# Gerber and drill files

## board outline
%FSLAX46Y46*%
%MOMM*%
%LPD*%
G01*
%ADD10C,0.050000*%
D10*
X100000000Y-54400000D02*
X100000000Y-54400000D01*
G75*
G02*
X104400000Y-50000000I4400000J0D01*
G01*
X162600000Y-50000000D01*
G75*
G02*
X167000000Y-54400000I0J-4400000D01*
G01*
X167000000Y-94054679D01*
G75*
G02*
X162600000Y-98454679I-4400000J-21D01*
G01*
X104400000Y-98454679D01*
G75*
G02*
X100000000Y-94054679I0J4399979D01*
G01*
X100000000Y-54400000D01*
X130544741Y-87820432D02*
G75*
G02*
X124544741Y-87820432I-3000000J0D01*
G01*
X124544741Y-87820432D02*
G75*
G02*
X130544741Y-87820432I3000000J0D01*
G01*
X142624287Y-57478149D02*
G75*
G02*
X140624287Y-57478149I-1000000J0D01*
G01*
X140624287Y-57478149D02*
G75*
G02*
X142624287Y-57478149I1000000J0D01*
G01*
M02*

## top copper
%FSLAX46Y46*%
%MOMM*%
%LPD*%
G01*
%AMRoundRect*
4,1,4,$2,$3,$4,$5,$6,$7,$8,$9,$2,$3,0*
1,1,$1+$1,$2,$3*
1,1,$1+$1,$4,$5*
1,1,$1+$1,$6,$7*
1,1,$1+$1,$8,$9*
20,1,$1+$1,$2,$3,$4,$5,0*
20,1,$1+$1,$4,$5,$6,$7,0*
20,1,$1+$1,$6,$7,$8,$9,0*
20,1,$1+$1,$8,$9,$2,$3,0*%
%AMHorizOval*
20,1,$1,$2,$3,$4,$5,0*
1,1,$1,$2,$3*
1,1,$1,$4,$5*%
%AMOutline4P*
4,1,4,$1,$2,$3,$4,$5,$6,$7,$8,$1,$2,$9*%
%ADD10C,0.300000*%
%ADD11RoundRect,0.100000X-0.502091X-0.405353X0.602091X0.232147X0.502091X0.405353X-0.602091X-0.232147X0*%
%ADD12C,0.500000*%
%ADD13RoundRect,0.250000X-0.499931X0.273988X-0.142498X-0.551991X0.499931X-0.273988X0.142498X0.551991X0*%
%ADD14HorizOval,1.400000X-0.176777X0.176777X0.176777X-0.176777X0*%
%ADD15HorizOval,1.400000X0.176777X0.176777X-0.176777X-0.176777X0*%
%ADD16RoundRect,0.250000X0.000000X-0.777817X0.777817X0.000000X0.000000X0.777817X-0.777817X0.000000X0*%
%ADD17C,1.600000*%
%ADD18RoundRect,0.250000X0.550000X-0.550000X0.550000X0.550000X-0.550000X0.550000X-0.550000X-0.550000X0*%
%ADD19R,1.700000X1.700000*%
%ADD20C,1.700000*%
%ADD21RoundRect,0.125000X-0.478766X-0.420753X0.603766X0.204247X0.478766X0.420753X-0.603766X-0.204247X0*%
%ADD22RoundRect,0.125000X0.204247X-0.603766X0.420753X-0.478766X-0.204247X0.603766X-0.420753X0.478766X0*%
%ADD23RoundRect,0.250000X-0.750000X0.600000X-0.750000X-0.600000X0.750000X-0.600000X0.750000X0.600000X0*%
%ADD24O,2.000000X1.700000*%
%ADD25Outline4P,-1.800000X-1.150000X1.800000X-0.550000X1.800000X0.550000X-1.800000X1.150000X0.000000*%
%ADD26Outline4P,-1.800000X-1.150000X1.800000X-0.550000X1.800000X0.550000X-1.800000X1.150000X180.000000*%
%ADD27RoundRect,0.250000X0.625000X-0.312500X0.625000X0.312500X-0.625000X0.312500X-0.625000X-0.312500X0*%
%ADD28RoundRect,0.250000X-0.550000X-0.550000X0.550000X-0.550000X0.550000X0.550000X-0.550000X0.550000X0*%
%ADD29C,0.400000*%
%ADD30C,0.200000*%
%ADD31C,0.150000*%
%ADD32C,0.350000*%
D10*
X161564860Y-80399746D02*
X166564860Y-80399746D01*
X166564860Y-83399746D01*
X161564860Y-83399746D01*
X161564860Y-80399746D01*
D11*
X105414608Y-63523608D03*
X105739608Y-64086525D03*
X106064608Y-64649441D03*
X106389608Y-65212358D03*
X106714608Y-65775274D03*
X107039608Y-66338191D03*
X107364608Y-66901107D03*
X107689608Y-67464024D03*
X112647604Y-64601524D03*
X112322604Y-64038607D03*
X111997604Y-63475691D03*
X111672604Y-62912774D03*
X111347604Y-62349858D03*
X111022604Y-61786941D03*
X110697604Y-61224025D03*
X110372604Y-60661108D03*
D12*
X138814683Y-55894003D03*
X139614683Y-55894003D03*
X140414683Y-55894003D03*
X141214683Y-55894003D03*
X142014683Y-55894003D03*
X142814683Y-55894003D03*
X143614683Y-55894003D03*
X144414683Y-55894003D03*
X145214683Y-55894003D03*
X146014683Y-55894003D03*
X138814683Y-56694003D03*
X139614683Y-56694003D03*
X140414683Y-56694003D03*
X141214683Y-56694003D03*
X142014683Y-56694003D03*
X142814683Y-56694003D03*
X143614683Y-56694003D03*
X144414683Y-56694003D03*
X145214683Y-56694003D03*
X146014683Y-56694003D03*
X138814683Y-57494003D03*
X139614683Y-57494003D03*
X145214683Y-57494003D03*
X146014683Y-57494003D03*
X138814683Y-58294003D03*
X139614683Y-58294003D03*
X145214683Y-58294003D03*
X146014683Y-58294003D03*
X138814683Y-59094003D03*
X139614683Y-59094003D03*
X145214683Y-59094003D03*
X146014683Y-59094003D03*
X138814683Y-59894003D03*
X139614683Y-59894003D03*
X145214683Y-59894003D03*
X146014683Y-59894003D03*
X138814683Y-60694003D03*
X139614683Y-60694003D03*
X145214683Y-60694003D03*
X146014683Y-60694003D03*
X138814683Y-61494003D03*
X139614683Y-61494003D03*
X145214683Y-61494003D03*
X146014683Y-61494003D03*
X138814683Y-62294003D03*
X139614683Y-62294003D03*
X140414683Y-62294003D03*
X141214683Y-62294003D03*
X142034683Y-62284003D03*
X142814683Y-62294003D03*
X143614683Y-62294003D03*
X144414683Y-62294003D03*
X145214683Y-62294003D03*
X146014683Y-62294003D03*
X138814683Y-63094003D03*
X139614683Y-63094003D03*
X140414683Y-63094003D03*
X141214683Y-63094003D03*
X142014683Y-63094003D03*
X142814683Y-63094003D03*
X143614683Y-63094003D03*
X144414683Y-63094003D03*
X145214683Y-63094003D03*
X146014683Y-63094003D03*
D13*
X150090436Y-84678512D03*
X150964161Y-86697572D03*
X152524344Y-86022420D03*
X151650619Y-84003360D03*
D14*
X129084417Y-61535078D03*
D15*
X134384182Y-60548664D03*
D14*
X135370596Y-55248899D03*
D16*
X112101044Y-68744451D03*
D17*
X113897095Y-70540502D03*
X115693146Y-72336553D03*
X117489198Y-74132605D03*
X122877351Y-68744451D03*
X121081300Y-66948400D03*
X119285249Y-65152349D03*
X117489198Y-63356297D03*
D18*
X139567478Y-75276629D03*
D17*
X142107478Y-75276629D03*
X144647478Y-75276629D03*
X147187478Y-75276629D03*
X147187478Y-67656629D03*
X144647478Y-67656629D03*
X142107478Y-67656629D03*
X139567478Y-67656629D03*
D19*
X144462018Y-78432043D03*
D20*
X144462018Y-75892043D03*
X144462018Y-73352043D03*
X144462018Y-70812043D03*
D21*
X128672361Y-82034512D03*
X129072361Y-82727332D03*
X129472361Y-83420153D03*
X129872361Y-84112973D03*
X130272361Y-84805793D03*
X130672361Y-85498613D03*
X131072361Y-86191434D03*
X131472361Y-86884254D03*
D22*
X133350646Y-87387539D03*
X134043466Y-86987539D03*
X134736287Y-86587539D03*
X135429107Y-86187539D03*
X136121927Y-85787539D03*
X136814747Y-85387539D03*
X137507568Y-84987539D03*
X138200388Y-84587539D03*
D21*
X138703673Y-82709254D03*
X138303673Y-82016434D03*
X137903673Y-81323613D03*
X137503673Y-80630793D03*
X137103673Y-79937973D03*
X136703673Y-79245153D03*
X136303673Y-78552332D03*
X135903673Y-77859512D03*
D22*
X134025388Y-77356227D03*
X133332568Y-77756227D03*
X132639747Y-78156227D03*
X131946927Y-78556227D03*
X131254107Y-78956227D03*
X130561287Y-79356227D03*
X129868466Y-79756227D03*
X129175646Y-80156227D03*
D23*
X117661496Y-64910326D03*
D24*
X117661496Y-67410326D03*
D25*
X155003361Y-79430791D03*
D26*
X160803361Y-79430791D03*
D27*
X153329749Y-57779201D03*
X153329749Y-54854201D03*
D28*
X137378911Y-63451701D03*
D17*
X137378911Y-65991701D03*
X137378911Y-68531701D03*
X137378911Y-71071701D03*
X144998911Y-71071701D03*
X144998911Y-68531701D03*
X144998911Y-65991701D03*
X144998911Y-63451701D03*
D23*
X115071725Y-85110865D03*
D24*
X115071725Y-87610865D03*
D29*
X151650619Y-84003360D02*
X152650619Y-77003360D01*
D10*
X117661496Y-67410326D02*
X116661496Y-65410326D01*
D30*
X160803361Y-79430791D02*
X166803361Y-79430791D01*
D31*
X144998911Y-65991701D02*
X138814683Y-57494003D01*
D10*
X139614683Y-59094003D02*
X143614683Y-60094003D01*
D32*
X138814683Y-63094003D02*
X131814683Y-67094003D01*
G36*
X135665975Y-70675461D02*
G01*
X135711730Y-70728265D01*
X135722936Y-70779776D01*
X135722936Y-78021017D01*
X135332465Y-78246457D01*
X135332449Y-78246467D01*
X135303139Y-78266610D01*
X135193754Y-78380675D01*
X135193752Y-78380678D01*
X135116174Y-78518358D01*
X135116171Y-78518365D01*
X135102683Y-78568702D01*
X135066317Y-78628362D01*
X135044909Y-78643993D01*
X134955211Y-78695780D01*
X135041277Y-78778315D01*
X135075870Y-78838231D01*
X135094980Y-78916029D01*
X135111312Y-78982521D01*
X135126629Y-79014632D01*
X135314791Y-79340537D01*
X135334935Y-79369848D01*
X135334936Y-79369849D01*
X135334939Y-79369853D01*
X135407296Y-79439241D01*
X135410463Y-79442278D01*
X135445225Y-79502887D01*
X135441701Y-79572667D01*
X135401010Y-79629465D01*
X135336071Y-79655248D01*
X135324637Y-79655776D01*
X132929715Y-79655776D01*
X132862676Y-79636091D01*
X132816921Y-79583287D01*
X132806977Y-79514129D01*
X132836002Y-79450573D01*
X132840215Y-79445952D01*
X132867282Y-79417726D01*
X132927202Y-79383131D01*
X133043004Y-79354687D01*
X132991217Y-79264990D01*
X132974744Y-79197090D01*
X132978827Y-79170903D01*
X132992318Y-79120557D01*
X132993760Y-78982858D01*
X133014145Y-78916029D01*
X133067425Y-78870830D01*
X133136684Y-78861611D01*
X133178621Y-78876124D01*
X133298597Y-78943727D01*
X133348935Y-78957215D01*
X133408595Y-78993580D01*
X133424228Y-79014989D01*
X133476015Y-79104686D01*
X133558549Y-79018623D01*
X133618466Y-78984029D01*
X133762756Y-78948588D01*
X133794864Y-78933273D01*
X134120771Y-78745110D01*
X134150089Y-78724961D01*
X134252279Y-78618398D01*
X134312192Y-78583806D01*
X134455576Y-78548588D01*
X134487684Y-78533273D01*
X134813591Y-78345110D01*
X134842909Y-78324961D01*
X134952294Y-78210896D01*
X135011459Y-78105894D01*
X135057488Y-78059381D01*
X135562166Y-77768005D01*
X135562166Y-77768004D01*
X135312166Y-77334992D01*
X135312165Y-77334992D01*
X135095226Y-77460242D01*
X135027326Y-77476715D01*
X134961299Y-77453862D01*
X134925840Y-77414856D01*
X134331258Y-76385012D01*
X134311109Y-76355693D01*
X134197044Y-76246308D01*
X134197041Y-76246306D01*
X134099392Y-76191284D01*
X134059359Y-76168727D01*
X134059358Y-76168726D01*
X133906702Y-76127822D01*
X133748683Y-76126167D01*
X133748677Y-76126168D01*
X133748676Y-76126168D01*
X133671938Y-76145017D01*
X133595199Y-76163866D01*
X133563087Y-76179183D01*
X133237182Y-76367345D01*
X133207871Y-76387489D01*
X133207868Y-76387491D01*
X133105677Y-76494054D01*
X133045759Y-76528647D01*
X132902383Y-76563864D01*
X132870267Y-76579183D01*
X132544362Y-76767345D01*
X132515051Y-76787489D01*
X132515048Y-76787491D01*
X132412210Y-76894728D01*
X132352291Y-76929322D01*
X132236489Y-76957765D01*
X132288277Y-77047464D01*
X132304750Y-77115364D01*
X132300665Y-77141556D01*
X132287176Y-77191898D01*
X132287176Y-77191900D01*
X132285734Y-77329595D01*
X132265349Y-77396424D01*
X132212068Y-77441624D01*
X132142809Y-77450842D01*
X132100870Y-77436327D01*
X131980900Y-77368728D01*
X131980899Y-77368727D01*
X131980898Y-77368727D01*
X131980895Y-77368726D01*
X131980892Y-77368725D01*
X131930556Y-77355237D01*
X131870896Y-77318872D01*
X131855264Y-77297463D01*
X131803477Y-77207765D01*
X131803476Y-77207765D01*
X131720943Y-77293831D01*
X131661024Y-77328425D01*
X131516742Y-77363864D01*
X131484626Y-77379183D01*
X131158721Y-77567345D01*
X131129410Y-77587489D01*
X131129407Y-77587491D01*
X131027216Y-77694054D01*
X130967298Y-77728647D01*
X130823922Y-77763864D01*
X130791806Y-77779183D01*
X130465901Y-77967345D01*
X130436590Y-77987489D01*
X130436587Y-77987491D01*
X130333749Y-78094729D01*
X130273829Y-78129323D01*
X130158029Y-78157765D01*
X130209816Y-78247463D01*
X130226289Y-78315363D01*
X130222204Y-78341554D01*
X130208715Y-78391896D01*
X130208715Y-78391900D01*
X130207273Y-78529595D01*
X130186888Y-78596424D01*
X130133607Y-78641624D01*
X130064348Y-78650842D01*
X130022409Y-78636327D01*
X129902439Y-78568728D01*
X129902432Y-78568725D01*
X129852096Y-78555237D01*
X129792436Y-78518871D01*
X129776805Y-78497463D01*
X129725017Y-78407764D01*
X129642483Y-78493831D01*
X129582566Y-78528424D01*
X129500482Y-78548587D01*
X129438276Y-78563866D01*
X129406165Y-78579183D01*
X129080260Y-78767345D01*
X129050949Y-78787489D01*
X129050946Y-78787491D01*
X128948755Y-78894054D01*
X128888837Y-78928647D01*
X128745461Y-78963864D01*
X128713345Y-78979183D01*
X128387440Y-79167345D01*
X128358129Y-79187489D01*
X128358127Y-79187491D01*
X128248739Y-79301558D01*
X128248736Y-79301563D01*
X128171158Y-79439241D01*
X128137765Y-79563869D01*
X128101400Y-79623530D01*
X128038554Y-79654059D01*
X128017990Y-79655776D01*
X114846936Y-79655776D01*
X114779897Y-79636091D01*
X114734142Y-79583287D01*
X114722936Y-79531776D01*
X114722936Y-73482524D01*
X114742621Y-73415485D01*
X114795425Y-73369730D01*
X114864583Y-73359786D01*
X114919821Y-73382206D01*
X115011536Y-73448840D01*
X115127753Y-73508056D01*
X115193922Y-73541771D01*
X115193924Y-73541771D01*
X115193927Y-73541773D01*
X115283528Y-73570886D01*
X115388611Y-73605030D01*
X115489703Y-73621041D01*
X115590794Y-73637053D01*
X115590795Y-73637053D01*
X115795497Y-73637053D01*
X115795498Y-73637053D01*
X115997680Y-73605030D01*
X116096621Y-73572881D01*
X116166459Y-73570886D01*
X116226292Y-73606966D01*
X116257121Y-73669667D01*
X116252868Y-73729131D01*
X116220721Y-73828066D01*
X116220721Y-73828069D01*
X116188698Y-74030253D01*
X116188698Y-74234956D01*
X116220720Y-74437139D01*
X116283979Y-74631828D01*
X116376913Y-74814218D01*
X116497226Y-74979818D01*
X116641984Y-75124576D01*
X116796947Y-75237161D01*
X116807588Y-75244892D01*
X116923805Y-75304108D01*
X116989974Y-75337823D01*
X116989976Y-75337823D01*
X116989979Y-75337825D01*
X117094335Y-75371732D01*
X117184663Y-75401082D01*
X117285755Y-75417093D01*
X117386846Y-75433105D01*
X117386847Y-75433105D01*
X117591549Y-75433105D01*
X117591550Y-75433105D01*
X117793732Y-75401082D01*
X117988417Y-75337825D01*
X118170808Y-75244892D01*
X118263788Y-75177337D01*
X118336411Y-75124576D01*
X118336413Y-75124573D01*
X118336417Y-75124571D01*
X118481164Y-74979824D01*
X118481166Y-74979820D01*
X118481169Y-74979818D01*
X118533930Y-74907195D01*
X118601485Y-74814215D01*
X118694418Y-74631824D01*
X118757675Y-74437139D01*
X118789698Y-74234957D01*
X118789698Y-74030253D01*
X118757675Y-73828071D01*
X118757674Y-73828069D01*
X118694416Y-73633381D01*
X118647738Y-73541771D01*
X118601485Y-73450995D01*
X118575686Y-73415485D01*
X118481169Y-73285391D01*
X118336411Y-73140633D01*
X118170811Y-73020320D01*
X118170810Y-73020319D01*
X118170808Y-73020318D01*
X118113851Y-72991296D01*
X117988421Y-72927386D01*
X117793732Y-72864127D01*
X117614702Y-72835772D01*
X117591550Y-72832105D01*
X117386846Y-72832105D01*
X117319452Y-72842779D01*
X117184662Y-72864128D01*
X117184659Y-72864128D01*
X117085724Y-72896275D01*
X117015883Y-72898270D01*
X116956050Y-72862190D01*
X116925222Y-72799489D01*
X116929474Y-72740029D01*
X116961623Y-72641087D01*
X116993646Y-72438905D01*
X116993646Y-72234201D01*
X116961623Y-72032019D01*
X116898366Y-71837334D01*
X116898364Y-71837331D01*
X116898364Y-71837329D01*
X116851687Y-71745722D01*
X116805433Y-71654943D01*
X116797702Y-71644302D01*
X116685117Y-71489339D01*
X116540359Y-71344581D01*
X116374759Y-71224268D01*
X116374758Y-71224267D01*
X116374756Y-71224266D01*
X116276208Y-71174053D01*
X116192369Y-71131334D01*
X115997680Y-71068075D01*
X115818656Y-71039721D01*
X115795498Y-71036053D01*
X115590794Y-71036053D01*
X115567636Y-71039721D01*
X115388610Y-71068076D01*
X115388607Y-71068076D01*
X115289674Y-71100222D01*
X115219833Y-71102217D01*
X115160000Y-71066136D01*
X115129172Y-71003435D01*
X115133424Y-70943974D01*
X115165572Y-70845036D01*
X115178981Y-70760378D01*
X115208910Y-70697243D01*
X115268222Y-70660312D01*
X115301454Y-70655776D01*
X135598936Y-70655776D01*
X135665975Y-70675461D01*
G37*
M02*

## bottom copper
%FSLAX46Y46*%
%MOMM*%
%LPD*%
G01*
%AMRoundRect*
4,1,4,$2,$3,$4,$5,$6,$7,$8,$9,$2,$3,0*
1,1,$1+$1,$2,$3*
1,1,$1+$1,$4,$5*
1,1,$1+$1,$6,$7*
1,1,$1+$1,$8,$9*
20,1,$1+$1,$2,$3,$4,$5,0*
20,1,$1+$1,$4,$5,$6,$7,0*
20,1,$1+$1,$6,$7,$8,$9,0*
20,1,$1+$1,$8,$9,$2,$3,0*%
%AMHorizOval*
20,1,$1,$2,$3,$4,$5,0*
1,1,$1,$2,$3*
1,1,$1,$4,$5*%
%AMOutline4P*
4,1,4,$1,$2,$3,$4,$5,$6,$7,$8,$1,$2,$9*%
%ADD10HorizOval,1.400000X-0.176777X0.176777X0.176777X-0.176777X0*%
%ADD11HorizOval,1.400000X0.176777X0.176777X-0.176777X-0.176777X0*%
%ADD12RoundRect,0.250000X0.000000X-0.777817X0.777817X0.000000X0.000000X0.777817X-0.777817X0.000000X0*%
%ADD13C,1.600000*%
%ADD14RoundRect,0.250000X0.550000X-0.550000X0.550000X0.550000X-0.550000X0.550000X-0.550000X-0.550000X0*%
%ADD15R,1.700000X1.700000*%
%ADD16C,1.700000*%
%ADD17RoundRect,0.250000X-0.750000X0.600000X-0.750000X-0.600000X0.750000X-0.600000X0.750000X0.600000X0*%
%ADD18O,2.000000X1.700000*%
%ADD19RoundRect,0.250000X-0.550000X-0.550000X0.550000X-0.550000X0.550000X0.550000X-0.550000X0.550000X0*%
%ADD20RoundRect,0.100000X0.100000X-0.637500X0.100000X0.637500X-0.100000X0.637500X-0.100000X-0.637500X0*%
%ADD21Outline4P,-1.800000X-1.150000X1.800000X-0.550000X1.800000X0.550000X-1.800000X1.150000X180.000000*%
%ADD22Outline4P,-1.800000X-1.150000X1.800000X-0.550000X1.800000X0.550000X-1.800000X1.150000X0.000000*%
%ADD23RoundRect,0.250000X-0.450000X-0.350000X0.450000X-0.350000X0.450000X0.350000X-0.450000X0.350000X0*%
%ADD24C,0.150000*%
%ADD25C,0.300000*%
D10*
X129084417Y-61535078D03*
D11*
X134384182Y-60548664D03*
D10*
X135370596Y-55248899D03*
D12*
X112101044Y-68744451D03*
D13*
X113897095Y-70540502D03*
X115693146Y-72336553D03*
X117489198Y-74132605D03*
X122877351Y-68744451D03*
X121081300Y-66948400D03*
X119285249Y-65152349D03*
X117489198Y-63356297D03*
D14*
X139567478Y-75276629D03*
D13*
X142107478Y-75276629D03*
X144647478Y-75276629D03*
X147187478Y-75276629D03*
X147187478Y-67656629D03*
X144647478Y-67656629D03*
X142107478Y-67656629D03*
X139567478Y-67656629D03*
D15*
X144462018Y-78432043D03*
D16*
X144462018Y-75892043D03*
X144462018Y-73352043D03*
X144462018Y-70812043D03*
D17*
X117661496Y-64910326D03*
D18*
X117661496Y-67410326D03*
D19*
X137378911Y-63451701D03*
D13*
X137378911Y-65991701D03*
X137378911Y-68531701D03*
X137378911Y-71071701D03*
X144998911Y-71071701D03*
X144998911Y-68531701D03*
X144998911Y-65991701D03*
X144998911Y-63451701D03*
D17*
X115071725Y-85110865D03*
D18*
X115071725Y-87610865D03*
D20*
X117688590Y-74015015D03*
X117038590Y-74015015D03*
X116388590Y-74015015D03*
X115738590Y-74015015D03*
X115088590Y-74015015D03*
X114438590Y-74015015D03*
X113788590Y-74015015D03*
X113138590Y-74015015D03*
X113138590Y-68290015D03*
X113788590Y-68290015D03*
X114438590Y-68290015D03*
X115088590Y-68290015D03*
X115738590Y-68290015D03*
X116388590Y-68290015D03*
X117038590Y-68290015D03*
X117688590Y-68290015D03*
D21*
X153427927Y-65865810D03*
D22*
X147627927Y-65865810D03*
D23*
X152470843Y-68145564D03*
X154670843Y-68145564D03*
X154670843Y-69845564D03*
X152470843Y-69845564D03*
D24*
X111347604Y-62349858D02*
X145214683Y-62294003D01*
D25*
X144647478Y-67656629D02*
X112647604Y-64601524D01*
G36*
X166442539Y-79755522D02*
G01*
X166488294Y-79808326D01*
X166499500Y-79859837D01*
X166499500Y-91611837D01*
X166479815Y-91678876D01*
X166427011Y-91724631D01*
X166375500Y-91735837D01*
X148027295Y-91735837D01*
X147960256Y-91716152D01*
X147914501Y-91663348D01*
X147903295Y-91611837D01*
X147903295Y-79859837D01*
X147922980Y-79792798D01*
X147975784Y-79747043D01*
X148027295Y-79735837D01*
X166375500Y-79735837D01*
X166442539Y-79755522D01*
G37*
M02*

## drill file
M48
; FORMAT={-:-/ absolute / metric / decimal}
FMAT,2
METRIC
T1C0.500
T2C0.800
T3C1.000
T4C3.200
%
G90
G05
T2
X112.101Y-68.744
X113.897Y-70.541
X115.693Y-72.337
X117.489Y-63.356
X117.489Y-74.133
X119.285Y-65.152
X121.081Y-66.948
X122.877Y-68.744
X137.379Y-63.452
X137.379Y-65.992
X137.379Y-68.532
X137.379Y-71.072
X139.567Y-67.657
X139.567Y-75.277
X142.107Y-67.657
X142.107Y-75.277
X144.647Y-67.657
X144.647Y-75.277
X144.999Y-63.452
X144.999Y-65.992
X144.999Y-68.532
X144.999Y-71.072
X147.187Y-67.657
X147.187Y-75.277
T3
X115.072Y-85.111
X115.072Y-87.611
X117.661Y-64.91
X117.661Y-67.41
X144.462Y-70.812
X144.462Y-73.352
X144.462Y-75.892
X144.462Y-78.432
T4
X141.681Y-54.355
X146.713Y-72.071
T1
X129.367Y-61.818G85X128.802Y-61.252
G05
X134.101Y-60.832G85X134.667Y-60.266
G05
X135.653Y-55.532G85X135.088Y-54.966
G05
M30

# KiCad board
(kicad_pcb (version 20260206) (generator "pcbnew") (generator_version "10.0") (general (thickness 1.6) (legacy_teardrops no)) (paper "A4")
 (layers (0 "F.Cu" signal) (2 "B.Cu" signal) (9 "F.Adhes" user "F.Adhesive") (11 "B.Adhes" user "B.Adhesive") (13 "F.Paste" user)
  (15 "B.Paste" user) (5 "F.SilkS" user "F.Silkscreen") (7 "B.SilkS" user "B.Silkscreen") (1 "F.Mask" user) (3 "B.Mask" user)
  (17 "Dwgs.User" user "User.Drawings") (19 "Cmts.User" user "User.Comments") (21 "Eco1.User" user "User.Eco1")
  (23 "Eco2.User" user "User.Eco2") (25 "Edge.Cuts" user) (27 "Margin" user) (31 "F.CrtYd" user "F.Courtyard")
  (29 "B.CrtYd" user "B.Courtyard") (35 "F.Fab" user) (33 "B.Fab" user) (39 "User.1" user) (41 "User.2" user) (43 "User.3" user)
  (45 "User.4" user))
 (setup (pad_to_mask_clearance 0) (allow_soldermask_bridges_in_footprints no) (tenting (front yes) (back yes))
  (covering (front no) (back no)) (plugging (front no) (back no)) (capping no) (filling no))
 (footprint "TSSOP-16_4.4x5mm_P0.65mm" (layer "F.Cu") (at 109.031106 64.062566 30)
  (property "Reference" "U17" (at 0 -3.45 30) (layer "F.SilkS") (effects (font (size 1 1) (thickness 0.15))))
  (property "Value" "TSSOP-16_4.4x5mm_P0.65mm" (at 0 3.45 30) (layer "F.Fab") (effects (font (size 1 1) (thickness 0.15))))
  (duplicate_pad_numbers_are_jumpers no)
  (pad "1" smd roundrect (at -2.8625 -2.275 30) (size 1.475 0.4) (layers "F.Cu" "F.Mask" "F.Paste") (roundrect_rratio 0.25))
  (pad "2" smd roundrect (at -2.8625 -1.625 30) (size 1.475 0.4) (layers "F.Cu" "F.Mask" "F.Paste") (roundrect_rratio 0.25) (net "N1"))
  (pad "3" smd roundrect (at -2.8625 -0.975 30) (size 1.475 0.4) (layers "F.Cu" "F.Mask" "F.Paste") (roundrect_rratio 0.25) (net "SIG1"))
  (pad "4" smd roundrect (at -2.8625 -0.325 30) (size 1.475 0.4) (layers "F.Cu" "F.Mask" "F.Paste") (roundrect_rratio 0.25) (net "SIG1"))
  (pad "5" smd roundrect (at -2.8625 0.325 30) (size 1.475 0.4) (layers "F.Cu" "F.Mask" "F.Paste") (roundrect_rratio 0.25) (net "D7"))
  (pad "6" smd roundrect (at -2.8625 0.975 30) (size 1.475 0.4) (layers "F.Cu" "F.Mask" "F.Paste") (roundrect_rratio 0.25) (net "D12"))
  (pad "7" smd roundrect (at -2.8625 1.625 30) (size 1.475 0.4) (layers "F.Cu" "F.Mask" "F.Paste") (roundrect_rratio 0.25))
  (pad "8" smd roundrect (at -2.8625 2.275 30) (size 1.475 0.4) (layers "F.Cu" "F.Mask" "F.Paste") (roundrect_rratio 0.25) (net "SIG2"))
  (pad "9" smd roundrect (at 2.8625 2.275 30) (size 1.475 0.4) (layers "F.Cu" "F.Mask" "F.Paste") (roundrect_rratio 0.25) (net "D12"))
  (pad "10" smd roundrect (at 2.8625 1.625 30) (size 1.475 0.4) (layers "F.Cu" "F.Mask" "F.Paste") (roundrect_rratio 0.25) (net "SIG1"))
  (pad "11" smd roundrect (at 2.8625 0.975 30) (size 1.475 0.4) (layers "F.Cu" "F.Mask" "F.Paste") (roundrect_rratio 0.25) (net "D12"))
  (pad "12" smd roundrect (at 2.8625 0.325 30) (size 1.475 0.4) (layers "F.Cu" "F.Mask" "F.Paste") (roundrect_rratio 0.25))
  (pad "13" smd roundrect (at 2.8625 -0.325 30) (size 1.475 0.4) (layers "F.Cu" "F.Mask" "F.Paste") (roundrect_rratio 0.25))
  (pad "14" smd roundrect (at 2.8625 -0.975 30) (size 1.475 0.4) (layers "F.Cu" "F.Mask" "F.Paste") (roundrect_rratio 0.25) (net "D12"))
  (pad "15" smd roundrect (at 2.8625 -1.625 30) (size 1.475 0.4) (layers "F.Cu" "F.Mask" "F.Paste") (roundrect_rratio 0.25) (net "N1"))
  (pad "16" smd roundrect (at 2.8625 -2.275 30) (size 1.475 0.4) (layers "F.Cu" "F.Mask" "F.Paste") (roundrect_rratio 0.25) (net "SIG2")))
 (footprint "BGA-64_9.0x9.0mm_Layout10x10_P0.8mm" (layer "F.Cu") (at 142.414683 59.494003)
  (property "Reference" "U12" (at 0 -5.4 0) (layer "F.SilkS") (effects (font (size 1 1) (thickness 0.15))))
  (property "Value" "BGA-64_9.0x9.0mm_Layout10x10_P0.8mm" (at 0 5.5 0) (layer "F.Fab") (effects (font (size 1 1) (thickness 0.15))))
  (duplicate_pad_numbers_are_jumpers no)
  (pad "A1" smd circle (at -3.6 -3.6) (size 0.5 0.5) (layers "F.Cu" "F.Mask" "F.Paste") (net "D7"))
  (pad "A2" smd circle (at -2.8 -3.6) (size 0.5 0.5) (layers "F.Cu" "F.Mask" "F.Paste") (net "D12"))
  (pad "A3" smd circle (at -2 -3.6) (size 0.5 0.5) (layers "F.Cu" "F.Mask" "F.Paste"))
  (pad "A4" smd circle (at -1.2 -3.6) (size 0.5 0.5) (layers "F.Cu" "F.Mask" "F.Paste") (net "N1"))
  (pad "A5" smd circle (at -0.4 -3.6) (size 0.5 0.5) (layers "F.Cu" "F.Mask" "F.Paste") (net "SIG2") (clearance 0.35))
  (pad "A6" smd circle (at 0.4 -3.6) (size 0.5 0.5) (layers "F.Cu" "F.Mask" "F.Paste"))
  (pad "A7" smd circle (at 1.2 -3.6) (size 0.5 0.5) (layers "F.Cu" "F.Mask" "F.Paste") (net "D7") (clearance 0.1))
  (pad "A8" smd circle (at 2 -3.6) (size 0.5 0.5) (layers "F.Cu" "F.Mask" "F.Paste") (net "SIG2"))
  (pad "A9" smd circle (at 2.8 -3.6) (size 0.5 0.5) (layers "F.Cu" "F.Mask" "F.Paste") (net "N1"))
  (pad "A10" smd circle (at 3.6 -3.6) (size 0.5 0.5) (layers "F.Cu" "F.Mask" "F.Paste"))
  (pad "B1" smd circle (at -3.6 -2.8) (size 0.5 0.5) (layers "F.Cu" "F.Mask" "F.Paste") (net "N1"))
  (pad "B2" smd circle (at -2.8 -2.8) (size 0.5 0.5) (layers "F.Cu" "F.Mask" "F.Paste") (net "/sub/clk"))
  (pad "B3" smd circle (at -2 -2.8) (size 0.5 0.5) (layers "F.Cu" "F.Mask" "F.Paste") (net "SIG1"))
  (pad "B4" smd circle (at -1.2 -2.8) (size 0.5 0.5) (layers "F.Cu" "F.Mask" "F.Paste"))
  (pad "B5" smd circle (at -0.4 -2.8) (size 0.5 0.5) (layers "F.Cu" "F.Mask" "F.Paste"))
  (pad "B6" smd circle (at 0.4 -2.8) (size 0.5 0.5) (layers "F.Cu" "F.Mask" "F.Paste") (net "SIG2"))
  (pad "B7" smd circle (at 1.2 -2.8) (size 0.5 0.5) (layers "F.Cu" "F.Mask" "F.Paste"))
  (pad "B8" smd circle (at 2 -2.8) (size 0.5 0.5) (layers "F.Cu" "F.Mask" "F.Paste"))
  (pad "B9" smd circle (at 2.8 -2.8) (size 0.5 0.5) (layers "F.Cu" "F.Mask" "F.Paste"))
  (pad "B10" smd circle (at 3.6 -2.8) (size 0.5 0.5) (layers "F.Cu" "F.Mask" "F.Paste") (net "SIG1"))
  (pad "C1" smd circle (at -3.6 -2) (size 0.5 0.5) (layers "F.Cu" "F.Mask" "F.Paste") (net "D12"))
  (pad "C2" smd circle (at -2.8 -2) (size 0.5 0.5) (layers "F.Cu" "F.Mask" "F.Paste") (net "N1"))
  (pad "C9" smd circle (at 2.8 -2) (size 0.5 0.5) (layers "F.Cu" "F.Mask" "F.Paste"))
  (pad "C10" smd circle (at 3.6 -2) (size 0.5 0.5) (layers "F.Cu" "F.Mask" "F.Paste") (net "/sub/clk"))
  (pad "D1" smd circle (at -3.6 -1.2) (size 0.5 0.5) (layers "F.Cu" "F.Mask" "F.Paste") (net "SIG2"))
  (pad "D2" smd circle (at -2.8 -1.2) (size 0.5 0.5) (layers "F.Cu" "F.Mask" "F.Paste"))
  (pad "D9" smd circle (at 2.8 -1.2) (size 0.5 0.5) (layers "F.Cu" "F.Mask" "F.Paste") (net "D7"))
  (pad "D10" smd circle (at 3.6 -1.2) (size 0.5 0.5) (layers "F.Cu" "F.Mask" "F.Paste") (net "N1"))
  (pad "E1" smd circle (at -3.6 -0.4) (size 0.5 0.5) (layers "F.Cu" "F.Mask" "F.Paste") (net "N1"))
  (pad "E2" smd circle (at -2.8 -0.4) (size 0.5 0.5) (layers "F.Cu" "F.Mask" "F.Paste") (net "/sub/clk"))
  (pad "E9" smd circle (at 2.8 -0.4) (size 0.5 0.5) (layers "F.Cu" "F.Mask" "F.Paste") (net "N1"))
  (pad "E10" smd circle (at 3.6 -0.4) (size 0.5 0.5) (layers "F.Cu" "F.Mask" "F.Paste"))
  (pad "F1" smd circle (at -3.6 0.4) (size 0.5 0.5) (layers "F.Cu" "F.Mask" "F.Paste") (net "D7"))
  (pad "F2" smd circle (at -2.8 0.4) (size 0.5 0.5) (layers "F.Cu" "F.Mask" "F.Paste") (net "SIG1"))
  (pad "F9" smd circle (at 2.8 0.4) (size 0.5 0.5) (layers "F.Cu" "F.Mask" "F.Paste"))
  (pad "F10" smd circle (at 3.6 0.4) (size 0.5 0.5) (layers "F.Cu" "F.Mask" "F.Paste") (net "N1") (clearance 0.1))
  (pad "G1" smd circle (at -3.6 1.2) (size 0.5 0.5) (layers "F.Cu" "F.Mask" "F.Paste") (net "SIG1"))
  (pad "G2" smd circle (at -2.8 1.2) (size 0.5 0.5) (layers "F.Cu" "F.Mask" "F.Paste"))
  (pad "G9" smd circle (at 2.8 1.2) (size 0.5 0.5) (layers "F.Cu" "F.Mask" "F.Paste"))
  (pad "G10" smd circle (at 3.6 1.2) (size 0.5 0.5) (layers "F.Cu" "F.Mask" "F.Paste"))
  (pad "H1" smd circle (at -3.6 2) (size 0.5 0.5) (layers "F.Cu" "F.Mask" "F.Paste") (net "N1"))
  (pad "H2" smd circle (at -2.8 2) (size 0.5 0.5) (layers "F.Cu" "F.Mask" "F.Paste"))
  (pad "H9" smd circle (at 2.8 2) (size 0.5 0.5) (layers "F.Cu" "F.Mask" "F.Paste") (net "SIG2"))
  (pad "H10" smd circle (at 3.6 2) (size 0.5 0.5) (layers "F.Cu" "F.Mask" "F.Paste") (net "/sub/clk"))
  (pad "J1" smd circle (at -3.6 2.8) (size 0.5 0.5) (layers "F.Cu" "F.Mask" "F.Paste") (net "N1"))
  (pad "J2" smd circle (at -2.8 2.8) (size 0.5 0.5) (layers "F.Cu" "F.Mask" "F.Paste") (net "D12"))
  (pad "J3" smd circle (at -2 2.8) (size 0.5 0.5) (layers "F.Cu" "F.Mask" "F.Paste") (clearance 0.35))
  (pad "J4" smd circle (at -1.2 2.8) (size 0.5 0.5) (layers "F.Cu" "F.Mask" "F.Paste") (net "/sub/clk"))
  (pad "J5" smd circle (at -0.38 2.79) (size 0.5 0.5) (layers "F.Cu" "F.Mask" "F.Paste") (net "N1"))
  (pad "J6" smd circle (at 0.4 2.8) (size 0.5 0.5) (layers "F.Cu" "F.Mask" "F.Paste") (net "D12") (clearance 0.35))
  (pad "J7" smd circle (at 1.2 2.8) (size 0.5 0.5) (layers "F.Cu" "F.Mask" "F.Paste"))
  (pad "J8" smd circle (at 2 2.8) (size 0.5 0.5) (layers "F.Cu" "F.Mask" "F.Paste") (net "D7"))
  (pad "J9" smd circle (at 2.8 2.8) (size 0.5 0.5) (layers "F.Cu" "F.Mask" "F.Paste") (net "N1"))
  (pad "J10" smd circle (at 3.6 2.8) (size 0.5 0.5) (layers "F.Cu" "F.Mask" "F.Paste") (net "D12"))
  (pad "K1" smd circle (at -3.6 3.6) (size 0.5 0.5) (layers "F.Cu" "F.Mask" "F.Paste") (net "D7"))
  (pad "K2" smd circle (at -2.8 3.6) (size 0.5 0.5) (layers "F.Cu" "F.Mask" "F.Paste"))
  (pad "K3" smd circle (at -2 3.6) (size 0.5 0.5) (layers "F.Cu" "F.Mask" "F.Paste") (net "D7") (clearance 0.35))
  (pad "K4" smd circle (at -1.2 3.6) (size 0.5 0.5) (layers "F.Cu" "F.Mask" "F.Paste") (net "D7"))
  (pad "K5" smd circle (at -0.4 3.6) (size 0.5 0.5) (layers "F.Cu" "F.Mask" "F.Paste") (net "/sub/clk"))
  (pad "K6" smd circle (at 0.4 3.6) (size 0.5 0.5) (layers "F.Cu" "F.Mask" "F.Paste") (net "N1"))
  (pad "K7" smd circle (at 1.2 3.6) (size 0.5 0.5) (layers "F.Cu" "F.Mask" "F.Paste"))
  (pad "K8" smd circle (at 2 3.6) (size 0.5 0.5) (layers "F.Cu" "F.Mask" "F.Paste") (clearance 0.1))
  (pad "K9" smd circle (at 2.8 3.6) (size 0.5 0.5) (layers "F.Cu" "F.Mask" "F.Paste") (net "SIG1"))
  (pad "K10" smd circle (at 3.6 3.6) (size 0.5 0.5) (layers "F.Cu" "F.Mask" "F.Paste") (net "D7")))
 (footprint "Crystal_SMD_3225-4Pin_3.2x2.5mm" (layer "F.Cu") (at 151.30739 85.350466 -66.6)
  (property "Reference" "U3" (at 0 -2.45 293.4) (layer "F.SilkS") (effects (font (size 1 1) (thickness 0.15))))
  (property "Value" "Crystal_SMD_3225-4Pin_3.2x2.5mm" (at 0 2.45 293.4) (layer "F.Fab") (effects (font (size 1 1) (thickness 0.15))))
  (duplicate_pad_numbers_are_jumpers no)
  (pad "1" smd roundrect (at -1.1 0.85 293.4) (size 1.4 1.2) (layers "F.Cu" "F.Mask" "F.Paste") (roundrect_rratio 0.208333) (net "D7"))
  (pad "2" smd roundrect (at 1.1 0.85 293.4) (size 1.4 1.2) (layers "F.Cu" "F.Mask" "F.Paste") (roundrect_rratio 0.208333))
  (pad "3" smd roundrect (at 1.1 -0.85 293.4) (size 1.4 1.2) (layers "F.Cu" "F.Mask" "F.Paste") (roundrect_rratio 0.208333) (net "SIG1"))
  (pad "4" smd roundrect (at -1.1 -0.85 293.4) (size 1.4 1.2) (layers "F.Cu" "F.Mask" "F.Paste") (roundrect_rratio 0.208333)))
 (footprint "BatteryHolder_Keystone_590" (layer "F.Cu") (at 134.384182 60.548664 45)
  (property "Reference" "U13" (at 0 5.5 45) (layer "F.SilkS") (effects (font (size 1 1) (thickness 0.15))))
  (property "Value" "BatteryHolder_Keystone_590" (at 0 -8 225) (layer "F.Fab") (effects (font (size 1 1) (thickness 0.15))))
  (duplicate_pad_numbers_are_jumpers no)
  (pad "1" thru_hole oval (at -4.445 -3.05 135) (size 1.9 1.4) (drill oval 1.3 0.5) (layers "*.Cu" "*.Mask") (remove_unused_layers no)
   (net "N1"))
  (pad "1" thru_hole oval (at 0 0 45) (size 1.9 1.4) (drill oval 1.3 0.5) (layers "*.Cu" "*.Mask") (remove_unused_layers no) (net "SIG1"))
  (pad "1" thru_hole oval (at 4.445 -3.05 135) (size 1.9 1.4) (drill oval 1.3 0.5) (layers "*.Cu" "*.Mask") (remove_unused_layers no)
   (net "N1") (clearance 0.35)))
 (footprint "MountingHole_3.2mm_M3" (layer "F.Cu") (at 146.713095 72.070667 45)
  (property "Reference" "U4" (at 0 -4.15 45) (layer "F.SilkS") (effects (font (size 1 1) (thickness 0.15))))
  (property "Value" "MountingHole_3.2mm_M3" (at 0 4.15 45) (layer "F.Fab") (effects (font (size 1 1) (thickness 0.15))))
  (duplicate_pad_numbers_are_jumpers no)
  (pad "" np_thru_hole circle (at 0 0 45) (size 3.2 3.2) (drill 3.2) (layers "*.Cu" "*.Mask")))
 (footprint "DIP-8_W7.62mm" (layer "F.Cu") (at 112.101044 68.744451 45)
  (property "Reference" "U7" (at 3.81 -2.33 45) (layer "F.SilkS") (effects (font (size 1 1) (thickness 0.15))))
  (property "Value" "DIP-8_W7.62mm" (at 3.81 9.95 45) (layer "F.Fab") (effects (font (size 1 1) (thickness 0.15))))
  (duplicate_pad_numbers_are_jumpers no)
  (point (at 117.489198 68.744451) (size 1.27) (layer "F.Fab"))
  (pad "1" thru_hole roundrect (at 0 0 45) (size 1.6 1.6) (drill 0.8) (layers "*.Cu" "*.Mask") (remove_unused_layers no)
   (roundrect_rratio 0.15625) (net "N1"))
  (pad "2" thru_hole circle (at 0 2.54 45) (size 1.6 1.6) (drill 0.8) (layers "*.Cu" "*.Mask") (remove_unused_layers no))
  (pad "3" thru_hole circle (at 0 5.079999 45) (size 1.6 1.6) (drill 0.8) (layers "*.Cu" "*.Mask") (remove_unused_layers no) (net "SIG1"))
  (pad "4" thru_hole circle (at 0 7.62 45) (size 1.6 1.6) (drill 0.8) (layers "*.Cu" "*.Mask") (remove_unused_layers no) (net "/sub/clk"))
  (pad "5" thru_hole circle (at 7.62 7.62 45) (size 1.6 1.6) (drill 0.8) (layers "*.Cu" "*.Mask") (remove_unused_layers no) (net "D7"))
  (pad "6" thru_hole circle (at 7.62 5.08 45) (size 1.6 1.6) (drill 0.8) (layers "*.Cu" "*.Mask") (remove_unused_layers no))
  (pad "7" thru_hole circle (at 7.62 2.54 45) (size 1.6 1.6) (drill 0.8) (layers "*.Cu" "*.Mask") (remove_unused_layers no) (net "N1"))
  (pad "8" thru_hole circle (at 7.62 0 45) (size 1.6 1.6) (drill 0.8) (layers "*.Cu" "*.Mask") (remove_unused_layers no) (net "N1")))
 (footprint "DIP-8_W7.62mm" (layer "F.Cu") (at 139.567478 75.276629 90)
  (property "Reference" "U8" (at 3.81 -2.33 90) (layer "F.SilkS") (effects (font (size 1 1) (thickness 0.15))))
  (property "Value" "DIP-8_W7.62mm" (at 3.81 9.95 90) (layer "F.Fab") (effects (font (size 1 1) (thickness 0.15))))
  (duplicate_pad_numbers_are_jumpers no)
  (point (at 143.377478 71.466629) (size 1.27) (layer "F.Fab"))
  (pad "1" thru_hole roundrect (at 0 0 90) (size 1.6 1.6) (drill 0.8) (layers "*.Cu" "*.Mask") (remove_unused_layers no)
   (roundrect_rratio 0.15625))
  (pad "2" thru_hole circle (at 0 2.54 90) (size 1.6 1.6) (drill 0.8) (layers "*.Cu" "*.Mask") (remove_unused_layers no) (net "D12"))
  (pad "3" thru_hole circle (at 0 5.08 90) (size 1.6 1.6) (drill 0.8) (layers "*.Cu" "*.Mask") (remove_unused_layers no) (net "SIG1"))
  (pad "4" thru_hole circle (at 0 7.62 90) (size 1.6 1.6) (drill 0.8) (layers "*.Cu" "*.Mask") (remove_unused_layers no) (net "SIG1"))
  (pad "5" thru_hole circle (at 7.62 7.62 90) (size 1.6 1.6) (drill 0.8) (layers "*.Cu" "*.Mask") (remove_unused_layers no) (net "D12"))
  (pad "6" thru_hole circle (at 7.62 5.08 90) (size 1.6 1.6) (drill 0.8) (layers "*.Cu" "*.Mask") (remove_unused_layers no) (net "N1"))
  (pad "7" thru_hole circle (at 7.62 2.54 90) (size 1.6 1.6) (drill 0.8) (layers "*.Cu" "*.Mask") (remove_unused_layers no) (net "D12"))
  (pad "8" thru_hole circle (at 7.62 0 90) (size 1.6 1.6) (drill 0.8) (layers "*.Cu" "*.Mask") (remove_unused_layers no) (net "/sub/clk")))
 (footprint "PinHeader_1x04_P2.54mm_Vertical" (layer "F.Cu") (at 144.462018 78.432043 180)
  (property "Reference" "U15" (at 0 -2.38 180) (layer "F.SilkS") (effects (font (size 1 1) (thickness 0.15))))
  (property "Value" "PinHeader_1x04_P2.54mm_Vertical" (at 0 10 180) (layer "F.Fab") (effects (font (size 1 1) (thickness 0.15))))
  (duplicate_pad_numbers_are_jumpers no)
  (pad "1" thru_hole rect (at 0 0 180) (size 1.7 1.7) (drill 1) (layers "*.Cu" "*.Mask") (remove_unused_layers no) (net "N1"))
  (pad "2" thru_hole circle (at 0 2.54 180) (size 1.7 1.7) (drill 1) (layers "*.Cu" "*.Mask") (remove_unused_layers no) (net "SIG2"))
  (pad "3" thru_hole circle (at 0 5.08 180) (size 1.7 1.7) (drill 1) (layers "*.Cu" "*.Mask") (remove_unused_layers no))
  (pad "4" thru_hole circle (at 0 7.62 180) (size 1.7 1.7) (drill 1) (layers "*.Cu" "*.Mask") (remove_unused_layers no) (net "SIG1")))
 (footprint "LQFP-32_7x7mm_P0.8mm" (layer "F.Cu") (at 133.688017 82.371883 30)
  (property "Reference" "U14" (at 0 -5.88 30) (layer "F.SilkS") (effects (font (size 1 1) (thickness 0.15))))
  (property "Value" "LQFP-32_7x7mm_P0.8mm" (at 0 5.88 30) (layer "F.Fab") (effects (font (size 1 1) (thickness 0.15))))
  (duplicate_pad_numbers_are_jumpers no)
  (pad "1" smd roundrect (at -4.175 -2.8 30) (size 1.5 0.5) (layers "F.Cu" "F.Mask" "F.Paste") (roundrect_rratio 0.25) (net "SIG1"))
  (pad "2" smd roundrect (at -4.175 -2 30) (size 1.5 0.5) (layers "F.Cu" "F.Mask" "F.Paste") (roundrect_rratio 0.25) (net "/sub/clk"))
  (pad "3" smd roundrect (at -4.175 -1.2 30) (size 1.5 0.5) (layers "F.Cu" "F.Mask" "F.Paste") (roundrect_rratio 0.25) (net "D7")
   (clearance 0.35))
  (pad "4" smd roundrect (at -4.175 -0.4 30) (size 1.5 0.5) (layers "F.Cu" "F.Mask" "F.Paste") (roundrect_rratio 0.25) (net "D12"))
  (pad "5" smd roundrect (at -4.175 0.4 30) (size 1.5 0.5) (layers "F.Cu" "F.Mask" "F.Paste") (roundrect_rratio 0.25) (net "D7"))
  (pad "6" smd roundrect (at -4.175 1.2 30) (size 1.5 0.5) (layers "F.Cu" "F.Mask" "F.Paste") (roundrect_rratio 0.25))
  (pad "7" smd roundrect (at -4.175 2 30) (size 1.5 0.5) (layers "F.Cu" "F.Mask" "F.Paste") (roundrect_rratio 0.25) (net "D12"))
  (pad "8" smd roundrect (at -4.175 2.8 30) (size 1.5 0.5) (layers "F.Cu" "F.Mask" "F.Paste") (roundrect_rratio 0.25))
  (pad "9" smd roundrect (at -2.8 4.175 30) (size 0.5 1.5) (layers "F.Cu" "F.Mask" "F.Paste") (roundrect_rratio 0.25) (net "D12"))
  (pad "10" smd roundrect (at -2 4.175 30) (size 0.5 1.5) (layers "F.Cu" "F.Mask" "F.Paste") (roundrect_rratio 0.25))
  (pad "11" smd roundrect (at -1.2 4.175 30) (size 0.5 1.5) (layers "F.Cu" "F.Mask" "F.Paste") (roundrect_rratio 0.25) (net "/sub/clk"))
  (pad "12" smd roundrect (at -0.4 4.175 30) (size 0.5 1.5) (layers "F.Cu" "F.Mask" "F.Paste") (roundrect_rratio 0.25) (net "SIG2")
   (clearance 0.35))
  (pad "13" smd roundrect (at 0.4 4.175 30) (size 0.5 1.5) (layers "F.Cu" "F.Mask" "F.Paste") (roundrect_rratio 0.25) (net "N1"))
  (pad "14" smd roundrect (at 1.2 4.175 30) (size 0.5 1.5) (layers "F.Cu" "F.Mask" "F.Paste") (roundrect_rratio 0.25) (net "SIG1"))
  (pad "15" smd roundrect (at 2 4.175 30) (size 0.5 1.5) (layers "F.Cu" "F.Mask" "F.Paste") (roundrect_rratio 0.25) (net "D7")
   (clearance 0.35))
  (pad "16" smd roundrect (at 2.8 4.175 30) (size 0.5 1.5) (layers "F.Cu" "F.Mask" "F.Paste") (roundrect_rratio 0.25))
  (pad "17" smd roundrect (at 4.175 2.8 30) (size 1.5 0.5) (layers "F.Cu" "F.Mask" "F.Paste") (roundrect_rratio 0.25) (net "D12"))
  (pad "18" smd roundrect (at 4.175 2 30) (size 1.5 0.5) (layers "F.Cu" "F.Mask" "F.Paste") (roundrect_rratio 0.25) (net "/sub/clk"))
  (pad "19" smd roundrect (at 4.175 1.2 30) (size 1.5 0.5) (layers "F.Cu" "F.Mask" "F.Paste") (roundrect_rratio 0.25) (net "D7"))
  (pad "20" smd roundrect (at 4.175 0.4 30) (size 1.5 0.5) (layers "F.Cu" "F.Mask" "F.Paste") (roundrect_rratio 0.25) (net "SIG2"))
  (pad "21" smd roundrect (at 4.175 -0.4 30) (size 1.5 0.5) (layers "F.Cu" "F.Mask" "F.Paste") (roundrect_rratio 0.25) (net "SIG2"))
  (pad "22" smd roundrect (at 4.175 -1.2 30) (size 1.5 0.5) (layers "F.Cu" "F.Mask" "F.Paste") (roundrect_rratio 0.25) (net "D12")
   (clearance 0.1))
  (pad "23" smd roundrect (at 4.175 -2 30) (size 1.5 0.5) (layers "F.Cu" "F.Mask" "F.Paste") (roundrect_rratio 0.25) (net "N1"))
  (pad "24" smd roundrect (at 4.175 -2.8 30) (size 1.5 0.5) (layers "F.Cu" "F.Mask" "F.Paste") (roundrect_rratio 0.25) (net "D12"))
  (pad "25" smd roundrect (at 2.8 -4.175 30) (size 0.5 1.5) (layers "F.Cu" "F.Mask" "F.Paste") (roundrect_rratio 0.25) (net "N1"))
  (pad "26" smd roundrect (at 2 -4.175 30) (size 0.5 1.5) (layers "F.Cu" "F.Mask" "F.Paste") (roundrect_rratio 0.25) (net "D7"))
  (pad "27" smd roundrect (at 1.2 -4.175 30) (size 0.5 1.5) (layers "F.Cu" "F.Mask" "F.Paste") (roundrect_rratio 0.25) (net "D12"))
  (pad "28" smd roundrect (at 0.4 -4.175 30) (size 0.5 1.5) (layers "F.Cu" "F.Mask" "F.Paste") (roundrect_rratio 0.25) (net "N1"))
  (pad "29" smd roundrect (at -0.4 -4.175 30) (size 0.5 1.5) (layers "F.Cu" "F.Mask" "F.Paste") (roundrect_rratio 0.25) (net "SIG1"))
  (pad "30" smd roundrect (at -1.2 -4.175 30) (size 0.5 1.5) (layers "F.Cu" "F.Mask" "F.Paste") (roundrect_rratio 0.25) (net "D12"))
  (pad "31" smd roundrect (at -2 -4.175 30) (size 0.5 1.5) (layers "F.Cu" "F.Mask" "F.Paste") (roundrect_rratio 0.25) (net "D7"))
  (pad "32" smd roundrect (at -2.8 -4.175 30) (size 0.5 1.5) (layers "F.Cu" "F.Mask" "F.Paste") (roundrect_rratio 0.25)))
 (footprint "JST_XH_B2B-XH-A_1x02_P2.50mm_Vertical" (layer "F.Cu") (at 117.661496 64.910326 -90)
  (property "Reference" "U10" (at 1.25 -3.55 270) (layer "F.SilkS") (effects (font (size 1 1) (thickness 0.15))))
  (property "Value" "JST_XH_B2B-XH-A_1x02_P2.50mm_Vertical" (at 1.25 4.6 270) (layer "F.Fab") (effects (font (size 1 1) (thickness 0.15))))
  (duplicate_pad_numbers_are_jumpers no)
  (pad "1" thru_hole roundrect (at 0 0 270) (size 1.7 2) (drill 1) (layers "*.Cu" "*.Mask") (remove_unused_layers no)
   (roundrect_rratio 0.147059))
  (pad "2" thru_hole oval (at 2.5 0 270) (size 1.7 2) (drill 1) (layers "*.Cu" "*.Mask") (remove_unused_layers no) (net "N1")))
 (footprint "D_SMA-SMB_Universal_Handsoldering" (layer "F.Cu") (at 157.903361 79.430791)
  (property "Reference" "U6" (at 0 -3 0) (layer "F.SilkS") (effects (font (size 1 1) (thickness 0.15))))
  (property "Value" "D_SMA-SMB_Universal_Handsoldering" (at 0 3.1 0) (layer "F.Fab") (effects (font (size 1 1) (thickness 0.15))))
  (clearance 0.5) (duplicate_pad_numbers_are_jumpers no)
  (pad "1" smd trapezoid (at -2.9 0) (size 3.6 1.7) (rect_delta 0.6 0) (layers "F.Cu" "F.Mask" "F.Paste") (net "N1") (clearance 0.1))
  (pad "2" smd trapezoid (at 2.9 0 180) (size 3.6 1.7) (rect_delta 0.6 0) (layers "F.Cu" "F.Mask" "F.Paste") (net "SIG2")))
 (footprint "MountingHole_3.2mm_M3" (layer "F.Cu") (at 141.680598 54.355057 180)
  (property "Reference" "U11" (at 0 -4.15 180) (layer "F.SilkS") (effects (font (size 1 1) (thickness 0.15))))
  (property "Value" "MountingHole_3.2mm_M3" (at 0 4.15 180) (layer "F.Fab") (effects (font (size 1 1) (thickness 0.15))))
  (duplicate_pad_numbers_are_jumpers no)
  (pad "" np_thru_hole circle (at 0 0 180) (size 3.2 3.2) (drill 3.2) (layers "*.Cu" "*.Mask")))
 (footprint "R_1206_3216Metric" (layer "F.Cu") (at 153.329749 56.316701 90)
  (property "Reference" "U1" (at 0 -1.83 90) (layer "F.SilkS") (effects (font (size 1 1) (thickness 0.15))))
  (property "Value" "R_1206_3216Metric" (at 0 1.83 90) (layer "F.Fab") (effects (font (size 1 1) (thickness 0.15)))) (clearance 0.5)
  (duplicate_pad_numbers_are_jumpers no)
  (pad "1" smd roundrect (at -1.4625 0 90) (size 1.125 1.75) (layers "F.Cu" "F.Mask" "F.Paste") (roundrect_rratio 0.222222))
  (pad "2" smd roundrect (at 1.4625 0 90) (size 1.125 1.75) (layers "F.Cu" "F.Mask" "F.Paste") (roundrect_rratio 0.222222) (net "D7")))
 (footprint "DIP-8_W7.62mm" (layer "F.Cu") (at 137.378911 63.451701)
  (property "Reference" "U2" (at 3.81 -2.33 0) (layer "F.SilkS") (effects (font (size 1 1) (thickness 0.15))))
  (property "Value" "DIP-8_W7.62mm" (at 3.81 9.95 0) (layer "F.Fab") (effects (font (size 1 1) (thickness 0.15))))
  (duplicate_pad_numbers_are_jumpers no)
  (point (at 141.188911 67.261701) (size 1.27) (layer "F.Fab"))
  (pad "1" thru_hole roundrect (at 0 0) (size 1.6 1.6) (drill 0.8) (layers "*.Cu" "*.Mask") (remove_unused_layers no)
   (roundrect_rratio 0.15625) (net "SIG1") (clearance 0.1))
  (pad "2" thru_hole circle (at 0 2.54) (size 1.6 1.6) (drill 0.8) (layers "*.Cu" "*.Mask") (remove_unused_layers no) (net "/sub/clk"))
  (pad "3" thru_hole circle (at 0 5.08) (size 1.6 1.6) (drill 0.8) (layers "*.Cu" "*.Mask") (remove_unused_layers no) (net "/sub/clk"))
  (pad "4" thru_hole circle (at 0 7.62) (size 1.6 1.6) (drill 0.8) (layers "*.Cu" "*.Mask") (remove_unused_layers no) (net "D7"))
  (pad "5" thru_hole circle (at 7.62 7.62) (size 1.6 1.6) (drill 0.8) (layers "*.Cu" "*.Mask") (remove_unused_layers no))
  (pad "6" thru_hole circle (at 7.62 5.08) (size 1.6 1.6) (drill 0.8) (layers "*.Cu" "*.Mask") (remove_unused_layers no) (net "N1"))
  (pad "7" thru_hole circle (at 7.62 2.54) (size 1.6 1.6) (drill 0.8) (layers "*.Cu" "*.Mask") (remove_unused_layers no) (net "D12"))
  (pad "8" thru_hole circle (at 7.62 0) (size 1.6 1.6) (drill 0.8) (layers "*.Cu" "*.Mask") (remove_unused_layers no)))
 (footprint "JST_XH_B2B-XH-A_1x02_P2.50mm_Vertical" (layer "B.Cu") (at 115.071725 85.110865 -90)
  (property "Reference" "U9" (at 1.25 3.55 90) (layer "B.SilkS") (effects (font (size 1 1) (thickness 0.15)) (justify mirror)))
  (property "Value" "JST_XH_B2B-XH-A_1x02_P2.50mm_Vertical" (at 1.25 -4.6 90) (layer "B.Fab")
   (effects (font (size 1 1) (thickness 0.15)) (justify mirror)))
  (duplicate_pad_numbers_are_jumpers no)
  (pad "1" thru_hole roundrect (at 0 0 270) (size 1.7 2) (drill 1) (layers "*.Cu" "*.Mask") (remove_unused_layers no)
   (roundrect_rratio 0.147059))
  (pad "2" thru_hole oval (at 2.5 0 270) (size 1.7 2) (drill 1) (layers "*.Cu" "*.Mask") (remove_unused_layers no) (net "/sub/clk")))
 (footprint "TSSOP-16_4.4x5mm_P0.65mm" (layer "B.Cu") (at 115.41359 71.152515 90)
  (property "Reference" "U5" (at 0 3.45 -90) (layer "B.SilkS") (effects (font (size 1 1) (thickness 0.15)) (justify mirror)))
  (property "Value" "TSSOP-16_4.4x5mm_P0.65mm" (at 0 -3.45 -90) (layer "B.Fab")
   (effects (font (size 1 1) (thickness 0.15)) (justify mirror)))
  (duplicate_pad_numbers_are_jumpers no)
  (pad "1" smd roundrect (at -2.8625 2.275 90) (size 1.475 0.4) (layers "B.Cu" "B.Mask" "B.Paste") (roundrect_rratio 0.25))
  (pad "2" smd roundrect (at -2.8625 1.625 90) (size 1.475 0.4) (layers "B.Cu" "B.Mask" "B.Paste") (roundrect_rratio 0.25) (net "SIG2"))
  (pad "3" smd roundrect (at -2.8625 0.975 90) (size 1.475 0.4) (layers "B.Cu" "B.Mask" "B.Paste") (roundrect_rratio 0.25) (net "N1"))
  (pad "4" smd roundrect (at -2.8625 0.325 90) (size 1.475 0.4) (layers "B.Cu" "B.Mask" "B.Paste") (roundrect_rratio 0.25) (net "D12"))
  (pad "5" smd roundrect (at -2.8625 -0.325 90) (size 1.475 0.4) (layers "B.Cu" "B.Mask" "B.Paste") (roundrect_rratio 0.25) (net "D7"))
  (pad "6" smd roundrect (at -2.8625 -0.975 90) (size 1.475 0.4) (layers "B.Cu" "B.Mask" "B.Paste") (roundrect_rratio 0.25) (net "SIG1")
   (clearance 0.35))
  (pad "7" smd roundrect (at -2.8625 -1.625 90) (size 1.475 0.4) (layers "B.Cu" "B.Mask" "B.Paste") (roundrect_rratio 0.25))
  (pad "8" smd roundrect (at -2.8625 -2.275 90) (size 1.475 0.4) (layers "B.Cu" "B.Mask" "B.Paste") (roundrect_rratio 0.25) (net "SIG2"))
  (pad "9" smd roundrect (at 2.8625 -2.275 90) (size 1.475 0.4) (layers "B.Cu" "B.Mask" "B.Paste") (roundrect_rratio 0.25) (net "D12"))
  (pad "10" smd roundrect (at 2.8625 -1.625 90) (size 1.475 0.4) (layers "B.Cu" "B.Mask" "B.Paste") (roundrect_rratio 0.25) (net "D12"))
  (pad "11" smd roundrect (at 2.8625 -0.975 90) (size 1.475 0.4) (layers "B.Cu" "B.Mask" "B.Paste") (roundrect_rratio 0.25))
  (pad "12" smd roundrect (at 2.8625 -0.325 90) (size 1.475 0.4) (layers "B.Cu" "B.Mask" "B.Paste") (roundrect_rratio 0.25) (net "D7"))
  (pad "13" smd roundrect (at 2.8625 0.325 90) (size 1.475 0.4) (layers "B.Cu" "B.Mask" "B.Paste") (roundrect_rratio 0.25) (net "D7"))
  (pad "14" smd roundrect (at 2.8625 0.975 90) (size 1.475 0.4) (layers "B.Cu" "B.Mask" "B.Paste") (roundrect_rratio 0.25) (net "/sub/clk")
   (clearance 0.1))
  (pad "15" smd roundrect (at 2.8625 1.625 90) (size 1.475 0.4) (layers "B.Cu" "B.Mask" "B.Paste") (roundrect_rratio 0.25))
  (pad "16" smd roundrect (at 2.8625 2.275 90) (size 1.475 0.4) (layers "B.Cu" "B.Mask" "B.Paste") (roundrect_rratio 0.25)))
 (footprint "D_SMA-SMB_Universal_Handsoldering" (layer "B.Cu") (at 150.527927 65.86581 180)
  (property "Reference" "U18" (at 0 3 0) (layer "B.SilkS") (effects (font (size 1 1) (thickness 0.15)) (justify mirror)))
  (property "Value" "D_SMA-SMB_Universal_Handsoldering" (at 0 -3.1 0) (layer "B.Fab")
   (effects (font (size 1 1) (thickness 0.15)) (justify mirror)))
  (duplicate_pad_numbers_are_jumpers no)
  (pad "1" smd trapezoid (at -2.9 0 180) (size 3.6 1.7) (rect_delta 0.6 0) (layers "B.Cu" "B.Mask" "B.Paste"))
  (pad "2" smd trapezoid (at 2.9 0) (size 3.6 1.7) (rect_delta 0.6 0) (layers "B.Cu" "B.Mask" "B.Paste") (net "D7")))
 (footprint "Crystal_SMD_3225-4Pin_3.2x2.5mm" (layer "B.Cu") (at 153.570843 68.995564)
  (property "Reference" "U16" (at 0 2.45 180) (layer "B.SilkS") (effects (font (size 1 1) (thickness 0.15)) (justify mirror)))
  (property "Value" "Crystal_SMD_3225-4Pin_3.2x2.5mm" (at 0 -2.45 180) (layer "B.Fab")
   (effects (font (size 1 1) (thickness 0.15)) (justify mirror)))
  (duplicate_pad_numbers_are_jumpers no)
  (pad "1" smd roundrect (at -1.1 -0.85) (size 1.4 1.2) (layers "B.Cu" "B.Mask" "B.Paste") (roundrect_rratio 0.208333) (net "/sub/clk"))
  (pad "2" smd roundrect (at 1.1 -0.85) (size 1.4 1.2) (layers "B.Cu" "B.Mask" "B.Paste") (roundrect_rratio 0.208333) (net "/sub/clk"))
  (pad "3" smd roundrect (at 1.1 0.85) (size 1.4 1.2) (layers "B.Cu" "B.Mask" "B.Paste") (roundrect_rratio 0.208333) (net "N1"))
  (pad "4" smd roundrect (at -1.1 0.85) (size 1.4 1.2) (layers "B.Cu" "B.Mask" "B.Paste") (roundrect_rratio 0.208333) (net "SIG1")))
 (gr_rect (start 161.56486 80.399746) (end 166.56486 83.399746) (stroke (width 0.3) (type default)) (fill no) (layer "F.Cu") (net "SIG2"))
 (gr_rect (start 100 50) (end 167 98.454679) (radius 4.4) (stroke (width 0.05) (type default)) (fill no) (layer "Edge.Cuts"))
 (gr_circle (center 127.544741 87.820432) (end 130.544741 87.820432) (stroke (width 0.05) (type default)) (fill no) (layer "Edge.Cuts"))
 (gr_circle (center 141.624287 57.478149) (end 142.624287 57.478149) (stroke (width 0.05) (type default)) (fill no) (layer "Edge.Cuts"))
 (segment (start 151.650619 84.00336) (end 152.650619 77.00336) (width 0.4) (layer "F.Cu") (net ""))
 (segment (start 117.661496 67.410326) (end 116.661496 65.410326) (width 0.3) (layer "F.Cu") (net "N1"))
 (segment (start 111.347604 62.349858) (end 145.214683 62.294003) (width 0.15) (layer "B.Cu") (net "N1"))
 (segment (start 144.647478 67.656629) (end 112.647604 64.601524) (width 0.3) (layer "B.Cu") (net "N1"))
 (segment (start 160.803361 79.430791) (end 166.803361 79.430791) (width 0.2) (layer "F.Cu") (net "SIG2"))
 (segment (start 144.998911 65.991701) (end 138.814683 57.494003) (width 0.15) (layer "F.Cu") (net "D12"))
 (segment (start 139.614683 59.094003) (end 143.614683 60.094003) (width 0.3) (layer "F.Cu") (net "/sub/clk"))
 (segment (start 138.814683 63.094003) (end 131.814683 67.094003) (width 0.35) (layer "F.Cu") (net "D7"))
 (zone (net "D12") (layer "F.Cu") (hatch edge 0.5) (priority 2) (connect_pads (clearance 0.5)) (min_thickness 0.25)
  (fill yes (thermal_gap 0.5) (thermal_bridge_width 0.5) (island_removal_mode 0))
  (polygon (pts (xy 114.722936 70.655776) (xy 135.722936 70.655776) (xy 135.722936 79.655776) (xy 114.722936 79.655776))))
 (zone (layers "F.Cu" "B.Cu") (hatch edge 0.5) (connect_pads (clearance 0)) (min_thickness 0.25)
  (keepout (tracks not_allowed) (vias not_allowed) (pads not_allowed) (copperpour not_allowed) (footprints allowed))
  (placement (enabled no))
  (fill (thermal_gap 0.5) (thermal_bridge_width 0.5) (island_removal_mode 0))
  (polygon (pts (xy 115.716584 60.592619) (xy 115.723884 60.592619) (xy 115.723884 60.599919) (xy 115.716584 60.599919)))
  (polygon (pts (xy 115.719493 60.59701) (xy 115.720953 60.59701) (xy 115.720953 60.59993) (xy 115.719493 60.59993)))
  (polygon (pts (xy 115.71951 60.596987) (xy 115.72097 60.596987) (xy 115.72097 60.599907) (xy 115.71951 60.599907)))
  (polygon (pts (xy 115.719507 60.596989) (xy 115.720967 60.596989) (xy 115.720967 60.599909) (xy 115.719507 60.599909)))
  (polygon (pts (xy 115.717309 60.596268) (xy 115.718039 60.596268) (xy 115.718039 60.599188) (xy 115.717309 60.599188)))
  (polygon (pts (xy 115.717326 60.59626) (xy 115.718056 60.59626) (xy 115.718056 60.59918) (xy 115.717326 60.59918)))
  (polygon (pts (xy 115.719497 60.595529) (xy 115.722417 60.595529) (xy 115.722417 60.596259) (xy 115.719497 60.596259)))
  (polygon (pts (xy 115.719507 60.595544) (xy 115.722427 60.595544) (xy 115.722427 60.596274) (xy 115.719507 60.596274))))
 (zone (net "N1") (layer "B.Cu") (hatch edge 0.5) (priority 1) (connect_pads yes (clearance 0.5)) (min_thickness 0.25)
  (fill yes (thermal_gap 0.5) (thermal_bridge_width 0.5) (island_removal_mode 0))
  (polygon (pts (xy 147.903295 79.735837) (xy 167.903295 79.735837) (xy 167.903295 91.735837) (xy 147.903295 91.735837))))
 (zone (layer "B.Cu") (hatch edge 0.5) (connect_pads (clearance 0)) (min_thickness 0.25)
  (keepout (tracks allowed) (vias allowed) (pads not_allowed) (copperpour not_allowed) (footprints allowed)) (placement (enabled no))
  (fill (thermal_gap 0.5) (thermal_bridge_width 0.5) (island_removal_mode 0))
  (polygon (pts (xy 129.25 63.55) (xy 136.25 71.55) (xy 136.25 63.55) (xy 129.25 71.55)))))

